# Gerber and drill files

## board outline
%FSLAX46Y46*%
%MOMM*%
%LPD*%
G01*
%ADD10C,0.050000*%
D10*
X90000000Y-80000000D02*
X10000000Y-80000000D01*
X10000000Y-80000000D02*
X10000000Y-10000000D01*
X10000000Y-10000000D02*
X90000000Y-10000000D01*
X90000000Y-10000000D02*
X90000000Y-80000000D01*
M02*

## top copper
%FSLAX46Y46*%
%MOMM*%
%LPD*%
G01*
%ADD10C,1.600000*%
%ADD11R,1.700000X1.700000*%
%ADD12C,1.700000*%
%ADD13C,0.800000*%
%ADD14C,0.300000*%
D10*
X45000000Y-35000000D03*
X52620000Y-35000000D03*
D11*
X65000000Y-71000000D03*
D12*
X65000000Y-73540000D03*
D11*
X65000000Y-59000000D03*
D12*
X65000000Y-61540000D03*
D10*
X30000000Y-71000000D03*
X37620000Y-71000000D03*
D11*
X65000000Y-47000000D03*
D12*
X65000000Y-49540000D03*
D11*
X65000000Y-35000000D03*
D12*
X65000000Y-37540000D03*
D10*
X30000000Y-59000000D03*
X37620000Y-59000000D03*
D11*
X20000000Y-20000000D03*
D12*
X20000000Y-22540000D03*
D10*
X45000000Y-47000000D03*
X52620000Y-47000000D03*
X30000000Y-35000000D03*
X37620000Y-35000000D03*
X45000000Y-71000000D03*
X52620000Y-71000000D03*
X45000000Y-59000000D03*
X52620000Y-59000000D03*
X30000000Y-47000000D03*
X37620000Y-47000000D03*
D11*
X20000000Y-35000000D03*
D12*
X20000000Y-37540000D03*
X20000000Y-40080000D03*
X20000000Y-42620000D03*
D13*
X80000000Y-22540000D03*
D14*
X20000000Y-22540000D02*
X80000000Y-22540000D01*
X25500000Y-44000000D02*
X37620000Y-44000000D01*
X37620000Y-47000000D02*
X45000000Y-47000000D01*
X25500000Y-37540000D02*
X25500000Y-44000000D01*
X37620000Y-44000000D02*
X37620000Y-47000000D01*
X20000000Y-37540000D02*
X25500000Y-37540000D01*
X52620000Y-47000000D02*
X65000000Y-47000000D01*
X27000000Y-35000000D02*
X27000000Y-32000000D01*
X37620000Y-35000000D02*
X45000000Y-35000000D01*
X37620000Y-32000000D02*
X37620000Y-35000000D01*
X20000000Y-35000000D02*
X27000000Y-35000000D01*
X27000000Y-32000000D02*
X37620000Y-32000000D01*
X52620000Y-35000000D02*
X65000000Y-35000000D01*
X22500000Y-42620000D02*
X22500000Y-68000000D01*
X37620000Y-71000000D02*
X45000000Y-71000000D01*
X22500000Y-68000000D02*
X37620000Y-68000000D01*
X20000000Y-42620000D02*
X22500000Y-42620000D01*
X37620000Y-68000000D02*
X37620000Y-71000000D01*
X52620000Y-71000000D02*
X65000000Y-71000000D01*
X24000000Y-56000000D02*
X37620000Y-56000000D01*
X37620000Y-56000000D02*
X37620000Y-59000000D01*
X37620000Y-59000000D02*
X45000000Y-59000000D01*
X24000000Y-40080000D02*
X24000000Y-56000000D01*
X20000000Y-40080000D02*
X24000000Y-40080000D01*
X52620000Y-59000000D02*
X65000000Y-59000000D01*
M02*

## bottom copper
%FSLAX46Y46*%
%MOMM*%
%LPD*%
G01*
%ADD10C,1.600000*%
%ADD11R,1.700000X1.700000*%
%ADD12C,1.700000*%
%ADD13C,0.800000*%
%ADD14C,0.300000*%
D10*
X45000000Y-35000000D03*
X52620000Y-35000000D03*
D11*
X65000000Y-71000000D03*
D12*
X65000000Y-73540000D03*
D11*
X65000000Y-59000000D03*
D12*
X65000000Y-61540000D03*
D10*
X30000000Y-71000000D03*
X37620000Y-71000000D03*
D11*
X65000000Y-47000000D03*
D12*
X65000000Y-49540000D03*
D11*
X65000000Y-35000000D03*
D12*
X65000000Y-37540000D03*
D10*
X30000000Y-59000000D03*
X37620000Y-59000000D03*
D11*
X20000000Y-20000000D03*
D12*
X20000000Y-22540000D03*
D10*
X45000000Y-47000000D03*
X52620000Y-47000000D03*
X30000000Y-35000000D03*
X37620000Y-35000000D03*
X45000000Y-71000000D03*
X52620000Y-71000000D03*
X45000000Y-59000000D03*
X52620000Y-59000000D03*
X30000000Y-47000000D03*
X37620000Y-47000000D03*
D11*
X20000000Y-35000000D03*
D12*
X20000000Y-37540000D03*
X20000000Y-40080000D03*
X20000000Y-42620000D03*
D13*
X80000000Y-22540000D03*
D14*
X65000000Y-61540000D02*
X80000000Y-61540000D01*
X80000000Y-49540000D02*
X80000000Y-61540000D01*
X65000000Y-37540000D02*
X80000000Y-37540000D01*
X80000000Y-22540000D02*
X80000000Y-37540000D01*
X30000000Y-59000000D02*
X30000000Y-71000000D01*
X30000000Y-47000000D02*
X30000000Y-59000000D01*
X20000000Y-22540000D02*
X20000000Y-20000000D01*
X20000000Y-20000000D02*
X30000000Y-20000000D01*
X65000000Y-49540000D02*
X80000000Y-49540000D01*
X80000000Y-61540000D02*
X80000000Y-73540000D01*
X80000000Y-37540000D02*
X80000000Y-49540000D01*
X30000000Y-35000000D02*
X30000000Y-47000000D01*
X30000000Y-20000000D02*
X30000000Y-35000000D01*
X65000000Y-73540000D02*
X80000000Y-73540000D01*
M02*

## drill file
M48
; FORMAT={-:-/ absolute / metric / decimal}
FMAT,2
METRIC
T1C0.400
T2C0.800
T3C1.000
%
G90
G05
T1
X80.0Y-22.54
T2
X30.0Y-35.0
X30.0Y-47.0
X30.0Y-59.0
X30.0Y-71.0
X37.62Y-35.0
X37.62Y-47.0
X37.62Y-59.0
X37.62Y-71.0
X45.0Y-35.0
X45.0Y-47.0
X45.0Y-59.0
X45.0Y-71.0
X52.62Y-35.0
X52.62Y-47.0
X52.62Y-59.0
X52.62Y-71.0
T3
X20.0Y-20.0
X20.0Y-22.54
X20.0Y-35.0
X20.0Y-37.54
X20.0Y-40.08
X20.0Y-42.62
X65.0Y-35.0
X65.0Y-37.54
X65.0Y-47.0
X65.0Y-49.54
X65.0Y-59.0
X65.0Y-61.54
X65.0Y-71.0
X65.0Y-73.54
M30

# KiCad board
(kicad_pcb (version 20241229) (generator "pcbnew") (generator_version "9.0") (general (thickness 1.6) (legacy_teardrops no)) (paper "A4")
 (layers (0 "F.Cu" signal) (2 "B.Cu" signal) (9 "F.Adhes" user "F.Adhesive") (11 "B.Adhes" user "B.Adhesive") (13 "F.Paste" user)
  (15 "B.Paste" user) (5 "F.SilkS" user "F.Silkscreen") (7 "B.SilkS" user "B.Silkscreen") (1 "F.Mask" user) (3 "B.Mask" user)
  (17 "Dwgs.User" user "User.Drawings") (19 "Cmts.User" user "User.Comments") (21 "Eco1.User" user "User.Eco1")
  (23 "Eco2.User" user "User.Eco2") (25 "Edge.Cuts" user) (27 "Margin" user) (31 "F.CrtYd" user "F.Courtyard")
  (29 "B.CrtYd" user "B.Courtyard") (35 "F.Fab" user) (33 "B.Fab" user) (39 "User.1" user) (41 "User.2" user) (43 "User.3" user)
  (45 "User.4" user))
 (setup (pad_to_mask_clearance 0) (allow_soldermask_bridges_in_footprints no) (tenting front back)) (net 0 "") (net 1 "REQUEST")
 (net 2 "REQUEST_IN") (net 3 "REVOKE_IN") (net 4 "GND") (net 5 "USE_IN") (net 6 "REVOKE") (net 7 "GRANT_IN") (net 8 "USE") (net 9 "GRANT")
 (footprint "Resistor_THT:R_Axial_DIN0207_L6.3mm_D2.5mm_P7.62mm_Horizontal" (layer "F.Cu") (at 45 35)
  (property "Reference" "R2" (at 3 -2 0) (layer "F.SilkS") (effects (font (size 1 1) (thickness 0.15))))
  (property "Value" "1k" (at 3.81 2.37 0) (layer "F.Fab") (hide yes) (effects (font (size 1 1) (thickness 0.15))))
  (pad "1" thru_hole circle (at 0 0) (size 1.6 1.6) (drill 0.8) (layers "*.Cu" "*.Mask") (remove_unused_layers no) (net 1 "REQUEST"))
  (pad "2" thru_hole circle (at 7.62 0) (size 1.6 1.6) (drill 0.8) (layers "*.Cu" "*.Mask") (remove_unused_layers no) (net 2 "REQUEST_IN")))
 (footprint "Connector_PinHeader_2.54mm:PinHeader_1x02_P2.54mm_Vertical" (layer "F.Cu") (at 65 71)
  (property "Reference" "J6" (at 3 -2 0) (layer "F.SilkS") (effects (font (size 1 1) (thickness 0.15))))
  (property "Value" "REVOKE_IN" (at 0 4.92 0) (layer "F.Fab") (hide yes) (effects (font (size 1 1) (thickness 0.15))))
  (pad "1" thru_hole rect (at 0 0) (size 1.7 1.7) (drill 1) (layers "*.Cu" "*.Mask") (remove_unused_layers no) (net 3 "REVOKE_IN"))
  (pad "2" thru_hole circle (at 0 2.54) (size 1.7 1.7) (drill 1) (layers "*.Cu" "*.Mask") (remove_unused_layers no) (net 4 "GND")))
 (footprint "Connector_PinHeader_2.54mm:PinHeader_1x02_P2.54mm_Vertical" (layer "F.Cu") (at 65 59)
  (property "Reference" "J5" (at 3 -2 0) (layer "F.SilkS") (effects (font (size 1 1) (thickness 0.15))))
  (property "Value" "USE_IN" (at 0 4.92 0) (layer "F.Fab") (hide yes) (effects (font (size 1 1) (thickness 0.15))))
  (pad "1" thru_hole rect (at 0 0) (size 1.7 1.7) (drill 1) (layers "*.Cu" "*.Mask") (remove_unused_layers no) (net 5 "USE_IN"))
  (pad "2" thru_hole circle (at 0 2.54) (size 1.7 1.7) (drill 1) (layers "*.Cu" "*.Mask") (remove_unused_layers no) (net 4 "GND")))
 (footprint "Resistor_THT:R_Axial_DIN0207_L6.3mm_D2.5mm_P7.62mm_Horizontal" (layer "F.Cu") (at 30 71)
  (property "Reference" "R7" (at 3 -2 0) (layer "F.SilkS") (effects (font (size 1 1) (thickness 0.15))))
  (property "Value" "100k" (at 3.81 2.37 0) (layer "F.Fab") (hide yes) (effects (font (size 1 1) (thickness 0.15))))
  (pad "1" thru_hole circle (at 0 0) (size 1.6 1.6) (drill 0.8) (layers "*.Cu" "*.Mask") (remove_unused_layers no) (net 4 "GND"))
  (pad "2" thru_hole circle (at 7.62 0) (size 1.6 1.6) (drill 0.8) (layers "*.Cu" "*.Mask") (remove_unused_layers no) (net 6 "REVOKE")))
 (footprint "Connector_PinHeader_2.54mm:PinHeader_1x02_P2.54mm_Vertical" (layer "F.Cu") (at 65 47)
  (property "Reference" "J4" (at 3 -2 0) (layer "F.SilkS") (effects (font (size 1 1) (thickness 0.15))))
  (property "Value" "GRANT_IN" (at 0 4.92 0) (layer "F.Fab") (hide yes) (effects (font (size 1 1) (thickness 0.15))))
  (pad "1" thru_hole rect (at 0 0) (size 1.7 1.7) (drill 1) (layers "*.Cu" "*.Mask") (remove_unused_layers no) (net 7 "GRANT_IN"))
  (pad "2" thru_hole circle (at 0 2.54) (size 1.7 1.7) (drill 1) (layers "*.Cu" "*.Mask") (remove_unused_layers no) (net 4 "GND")))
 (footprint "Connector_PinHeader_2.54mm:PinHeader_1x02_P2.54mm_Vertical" (layer "F.Cu") (at 65 35)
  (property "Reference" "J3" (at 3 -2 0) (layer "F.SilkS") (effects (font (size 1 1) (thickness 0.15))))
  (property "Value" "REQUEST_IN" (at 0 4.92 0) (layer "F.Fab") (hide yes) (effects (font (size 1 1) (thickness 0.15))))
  (pad "1" thru_hole rect (at 0 0) (size 1.7 1.7) (drill 1) (layers "*.Cu" "*.Mask") (remove_unused_layers no) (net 2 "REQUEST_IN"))
  (pad "2" thru_hole circle (at 0 2.54) (size 1.7 1.7) (drill 1) (layers "*.Cu" "*.Mask") (remove_unused_layers no) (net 4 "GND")))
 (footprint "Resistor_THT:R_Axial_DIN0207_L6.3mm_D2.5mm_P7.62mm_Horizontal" (layer "F.Cu") (at 30 59)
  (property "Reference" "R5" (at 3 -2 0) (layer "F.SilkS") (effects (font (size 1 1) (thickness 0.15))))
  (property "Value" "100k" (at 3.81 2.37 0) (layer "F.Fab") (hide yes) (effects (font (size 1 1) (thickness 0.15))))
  (pad "1" thru_hole circle (at 0 0) (size 1.6 1.6) (drill 0.8) (layers "*.Cu" "*.Mask") (remove_unused_layers no) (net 4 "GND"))
  (pad "2" thru_hole circle (at 7.62 0) (size 1.6 1.6) (drill 0.8) (layers "*.Cu" "*.Mask") (remove_unused_layers no) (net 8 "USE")))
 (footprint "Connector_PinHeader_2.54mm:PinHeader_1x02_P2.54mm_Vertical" (layer "F.Cu") (at 20 20)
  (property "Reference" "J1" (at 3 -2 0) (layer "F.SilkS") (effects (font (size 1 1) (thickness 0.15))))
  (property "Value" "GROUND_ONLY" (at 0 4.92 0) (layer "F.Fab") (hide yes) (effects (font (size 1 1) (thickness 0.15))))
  (pad "1" thru_hole rect (at 0 0) (size 1.7 1.7) (drill 1) (layers "*.Cu" "*.Mask") (remove_unused_layers no) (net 4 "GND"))
  (pad "2" thru_hole circle (at 0 2.54) (size 1.7 1.7) (drill 1) (layers "*.Cu" "*.Mask") (remove_unused_layers no) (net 4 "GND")))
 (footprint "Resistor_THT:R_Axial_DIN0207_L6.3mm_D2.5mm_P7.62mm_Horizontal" (layer "F.Cu") (at 45 47)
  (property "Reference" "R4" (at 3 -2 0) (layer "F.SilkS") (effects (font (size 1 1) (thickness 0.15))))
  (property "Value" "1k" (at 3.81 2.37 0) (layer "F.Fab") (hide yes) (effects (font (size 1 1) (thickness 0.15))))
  (pad "1" thru_hole circle (at 0 0) (size 1.6 1.6) (drill 0.8) (layers "*.Cu" "*.Mask") (remove_unused_layers no) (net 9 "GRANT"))
  (pad "2" thru_hole circle (at 7.62 0) (size 1.6 1.6) (drill 0.8) (layers "*.Cu" "*.Mask") (remove_unused_layers no) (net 7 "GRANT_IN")))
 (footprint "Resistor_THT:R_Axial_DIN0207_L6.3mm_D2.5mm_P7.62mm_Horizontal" (layer "F.Cu") (at 30 35)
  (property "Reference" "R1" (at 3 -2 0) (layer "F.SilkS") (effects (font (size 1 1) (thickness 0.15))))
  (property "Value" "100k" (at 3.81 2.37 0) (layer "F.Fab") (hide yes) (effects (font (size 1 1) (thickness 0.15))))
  (pad "1" thru_hole circle (at 0 0) (size 1.6 1.6) (drill 0.8) (layers "*.Cu" "*.Mask") (remove_unused_layers no) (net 4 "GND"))
  (pad "2" thru_hole circle (at 7.62 0) (size 1.6 1.6) (drill 0.8) (layers "*.Cu" "*.Mask") (remove_unused_layers no) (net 1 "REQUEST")))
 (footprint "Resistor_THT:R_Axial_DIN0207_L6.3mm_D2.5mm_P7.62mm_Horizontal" (layer "F.Cu") (at 45 71)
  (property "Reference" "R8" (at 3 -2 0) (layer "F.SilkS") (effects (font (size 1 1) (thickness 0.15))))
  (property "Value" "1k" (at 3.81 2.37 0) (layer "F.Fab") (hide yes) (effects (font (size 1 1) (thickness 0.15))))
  (pad "1" thru_hole circle (at 0 0) (size 1.6 1.6) (drill 0.8) (layers "*.Cu" "*.Mask") (remove_unused_layers no) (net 6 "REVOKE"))
  (pad "2" thru_hole circle (at 7.62 0) (size 1.6 1.6) (drill 0.8) (layers "*.Cu" "*.Mask") (remove_unused_layers no) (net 3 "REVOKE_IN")))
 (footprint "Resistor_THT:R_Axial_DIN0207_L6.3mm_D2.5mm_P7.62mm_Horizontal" (layer "F.Cu") (at 45 59)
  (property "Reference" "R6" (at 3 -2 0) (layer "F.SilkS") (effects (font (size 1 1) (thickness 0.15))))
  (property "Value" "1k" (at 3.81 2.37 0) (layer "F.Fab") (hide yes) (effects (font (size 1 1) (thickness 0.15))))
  (pad "1" thru_hole circle (at 0 0) (size 1.6 1.6) (drill 0.8) (layers "*.Cu" "*.Mask") (remove_unused_layers no) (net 8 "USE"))
  (pad "2" thru_hole circle (at 7.62 0) (size 1.6 1.6) (drill 0.8) (layers "*.Cu" "*.Mask") (remove_unused_layers no) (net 5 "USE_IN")))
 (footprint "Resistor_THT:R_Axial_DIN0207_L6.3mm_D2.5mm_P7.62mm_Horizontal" (layer "F.Cu") (at 30 47)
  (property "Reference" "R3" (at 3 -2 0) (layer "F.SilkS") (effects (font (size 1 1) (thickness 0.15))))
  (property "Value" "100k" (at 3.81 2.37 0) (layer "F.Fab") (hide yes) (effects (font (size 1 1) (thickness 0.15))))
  (pad "1" thru_hole circle (at 0 0) (size 1.6 1.6) (drill 0.8) (layers "*.Cu" "*.Mask") (remove_unused_layers no) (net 4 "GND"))
  (pad "2" thru_hole circle (at 7.62 0) (size 1.6 1.6) (drill 0.8) (layers "*.Cu" "*.Mask") (remove_unused_layers no) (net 9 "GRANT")))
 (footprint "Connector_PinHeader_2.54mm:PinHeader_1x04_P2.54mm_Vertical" (layer "F.Cu") (at 20 35)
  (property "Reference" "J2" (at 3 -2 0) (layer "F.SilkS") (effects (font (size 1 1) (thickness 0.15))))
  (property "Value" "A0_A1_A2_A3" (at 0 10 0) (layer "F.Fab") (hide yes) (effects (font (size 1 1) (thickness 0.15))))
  (pad "1" thru_hole rect (at 0 0) (size 1.7 1.7) (drill 1) (layers "*.Cu" "*.Mask") (remove_unused_layers no) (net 1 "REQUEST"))
  (pad "2" thru_hole circle (at 0 2.54) (size 1.7 1.7) (drill 1) (layers "*.Cu" "*.Mask") (remove_unused_layers no) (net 9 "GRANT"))
  (pad "3" thru_hole circle (at 0 5.08) (size 1.7 1.7) (drill 1) (layers "*.Cu" "*.Mask") (remove_unused_layers no) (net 8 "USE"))
  (pad "4" thru_hole circle (at 0 7.62) (size 1.7 1.7) (drill 1) (layers "*.Cu" "*.Mask") (remove_unused_layers no) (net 6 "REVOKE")))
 (gr_line (start 90 80) (end 10 80) (stroke (width 0.05) (type default)) (layer "Edge.Cuts"))
 (gr_line (start 10 80) (end 10 10) (stroke (width 0.05) (type default)) (layer "Edge.Cuts"))
 (gr_line (start 10 10) (end 90 10) (stroke (width 0.05) (type default)) (layer "Edge.Cuts"))
 (gr_line (start 90 10) (end 90 80) (stroke (width 0.05) (type default)) (layer "Edge.Cuts"))
 (segment (start 20 22.54) (end 80 22.54) (width 0.3) (layer "F.Cu") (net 4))
 (via (at 80 22.54) (size 0.8) (drill 0.4) (layers "F.Cu" "B.Cu") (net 4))
 (segment (start 65 61.54) (end 80 61.54) (width 0.3) (layer "B.Cu") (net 4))
 (segment (start 80 49.54) (end 80 61.54) (width 0.3) (layer "B.Cu") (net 4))
 (segment (start 65 37.54) (end 80 37.54) (width 0.3) (layer "B.Cu") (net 4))
 (segment (start 80 22.54) (end 80 37.54) (width 0.3) (layer "B.Cu") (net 4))
 (segment (start 30 59) (end 30 71) (width 0.3) (layer "B.Cu") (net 4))
 (segment (start 30 47) (end 30 59) (width 0.3) (layer "B.Cu") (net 4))
 (segment (start 20 22.54) (end 20 20) (width 0.3) (layer "B.Cu") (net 4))
 (segment (start 20 20) (end 30 20) (width 0.3) (layer "B.Cu") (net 4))
 (segment (start 65 49.54) (end 80 49.54) (width 0.3) (layer "B.Cu") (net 4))
 (segment (start 80 61.54) (end 80 73.54) (width 0.3) (layer "B.Cu") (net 4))
 (segment (start 80 37.54) (end 80 49.54) (width 0.3) (layer "B.Cu") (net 4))
 (segment (start 30 35) (end 30 47) (width 0.3) (layer "B.Cu") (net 4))
 (segment (start 30 20) (end 30 35) (width 0.3) (layer "B.Cu") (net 4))
 (segment (start 65 73.54) (end 80 73.54) (width 0.3) (layer "B.Cu") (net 4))
 (segment (start 25.5 44) (end 37.62 44) (width 0.3) (layer "F.Cu") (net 9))
 (segment (start 37.62 47) (end 45 47) (width 0.3) (layer "F.Cu") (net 9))
 (segment (start 25.5 37.54) (end 25.5 44) (width 0.3) (layer "F.Cu") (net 9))
 (segment (start 37.62 44) (end 37.62 47) (width 0.3) (layer "F.Cu") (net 9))
 (segment (start 20 37.54) (end 25.5 37.54) (width 0.3) (layer "F.Cu") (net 9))
 (segment (start 52.62 47) (end 65 47) (width 0.3) (layer "F.Cu") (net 7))
 (segment (start 27 35) (end 27 32) (width 0.3) (layer "F.Cu") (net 1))
 (segment (start 37.62 35) (end 45 35) (width 0.3) (layer "F.Cu") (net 1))
 (segment (start 37.62 32) (end 37.62 35) (width 0.3) (layer "F.Cu") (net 1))
 (segment (start 20 35) (end 27 35) (width 0.3) (layer "F.Cu") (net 1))
 (segment (start 27 32) (end 37.62 32) (width 0.3) (layer "F.Cu") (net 1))
 (segment (start 52.62 35) (end 65 35) (width 0.3) (layer "F.Cu") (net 2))
 (segment (start 22.5 42.62) (end 22.5 68) (width 0.3) (layer "F.Cu") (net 6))
 (segment (start 37.62 71) (end 45 71) (width 0.3) (layer "F.Cu") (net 6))
 (segment (start 22.5 68) (end 37.62 68) (width 0.3) (layer "F.Cu") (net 6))
 (segment (start 20 42.62) (end 22.5 42.62) (width 0.3) (layer "F.Cu") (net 6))
 (segment (start 37.62 68) (end 37.62 71) (width 0.3) (layer "F.Cu") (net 6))
 (segment (start 52.62 71) (end 65 71) (width 0.3) (layer "F.Cu") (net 3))
 (segment (start 24 56) (end 37.62 56) (width 0.3) (layer "F.Cu") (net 8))
 (segment (start 37.62 56) (end 37.62 59) (width 0.3) (layer "F.Cu") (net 8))
 (segment (start 37.62 59) (end 45 59) (width 0.3) (layer "F.Cu") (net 8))
 (segment (start 24 40.08) (end 24 56) (width 0.3) (layer "F.Cu") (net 8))
 (segment (start 20 40.08) (end 24 40.08) (width 0.3) (layer "F.Cu") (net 8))
 (segment (start 52.62 59) (end 65 59) (width 0.3) (layer "F.Cu") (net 5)))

